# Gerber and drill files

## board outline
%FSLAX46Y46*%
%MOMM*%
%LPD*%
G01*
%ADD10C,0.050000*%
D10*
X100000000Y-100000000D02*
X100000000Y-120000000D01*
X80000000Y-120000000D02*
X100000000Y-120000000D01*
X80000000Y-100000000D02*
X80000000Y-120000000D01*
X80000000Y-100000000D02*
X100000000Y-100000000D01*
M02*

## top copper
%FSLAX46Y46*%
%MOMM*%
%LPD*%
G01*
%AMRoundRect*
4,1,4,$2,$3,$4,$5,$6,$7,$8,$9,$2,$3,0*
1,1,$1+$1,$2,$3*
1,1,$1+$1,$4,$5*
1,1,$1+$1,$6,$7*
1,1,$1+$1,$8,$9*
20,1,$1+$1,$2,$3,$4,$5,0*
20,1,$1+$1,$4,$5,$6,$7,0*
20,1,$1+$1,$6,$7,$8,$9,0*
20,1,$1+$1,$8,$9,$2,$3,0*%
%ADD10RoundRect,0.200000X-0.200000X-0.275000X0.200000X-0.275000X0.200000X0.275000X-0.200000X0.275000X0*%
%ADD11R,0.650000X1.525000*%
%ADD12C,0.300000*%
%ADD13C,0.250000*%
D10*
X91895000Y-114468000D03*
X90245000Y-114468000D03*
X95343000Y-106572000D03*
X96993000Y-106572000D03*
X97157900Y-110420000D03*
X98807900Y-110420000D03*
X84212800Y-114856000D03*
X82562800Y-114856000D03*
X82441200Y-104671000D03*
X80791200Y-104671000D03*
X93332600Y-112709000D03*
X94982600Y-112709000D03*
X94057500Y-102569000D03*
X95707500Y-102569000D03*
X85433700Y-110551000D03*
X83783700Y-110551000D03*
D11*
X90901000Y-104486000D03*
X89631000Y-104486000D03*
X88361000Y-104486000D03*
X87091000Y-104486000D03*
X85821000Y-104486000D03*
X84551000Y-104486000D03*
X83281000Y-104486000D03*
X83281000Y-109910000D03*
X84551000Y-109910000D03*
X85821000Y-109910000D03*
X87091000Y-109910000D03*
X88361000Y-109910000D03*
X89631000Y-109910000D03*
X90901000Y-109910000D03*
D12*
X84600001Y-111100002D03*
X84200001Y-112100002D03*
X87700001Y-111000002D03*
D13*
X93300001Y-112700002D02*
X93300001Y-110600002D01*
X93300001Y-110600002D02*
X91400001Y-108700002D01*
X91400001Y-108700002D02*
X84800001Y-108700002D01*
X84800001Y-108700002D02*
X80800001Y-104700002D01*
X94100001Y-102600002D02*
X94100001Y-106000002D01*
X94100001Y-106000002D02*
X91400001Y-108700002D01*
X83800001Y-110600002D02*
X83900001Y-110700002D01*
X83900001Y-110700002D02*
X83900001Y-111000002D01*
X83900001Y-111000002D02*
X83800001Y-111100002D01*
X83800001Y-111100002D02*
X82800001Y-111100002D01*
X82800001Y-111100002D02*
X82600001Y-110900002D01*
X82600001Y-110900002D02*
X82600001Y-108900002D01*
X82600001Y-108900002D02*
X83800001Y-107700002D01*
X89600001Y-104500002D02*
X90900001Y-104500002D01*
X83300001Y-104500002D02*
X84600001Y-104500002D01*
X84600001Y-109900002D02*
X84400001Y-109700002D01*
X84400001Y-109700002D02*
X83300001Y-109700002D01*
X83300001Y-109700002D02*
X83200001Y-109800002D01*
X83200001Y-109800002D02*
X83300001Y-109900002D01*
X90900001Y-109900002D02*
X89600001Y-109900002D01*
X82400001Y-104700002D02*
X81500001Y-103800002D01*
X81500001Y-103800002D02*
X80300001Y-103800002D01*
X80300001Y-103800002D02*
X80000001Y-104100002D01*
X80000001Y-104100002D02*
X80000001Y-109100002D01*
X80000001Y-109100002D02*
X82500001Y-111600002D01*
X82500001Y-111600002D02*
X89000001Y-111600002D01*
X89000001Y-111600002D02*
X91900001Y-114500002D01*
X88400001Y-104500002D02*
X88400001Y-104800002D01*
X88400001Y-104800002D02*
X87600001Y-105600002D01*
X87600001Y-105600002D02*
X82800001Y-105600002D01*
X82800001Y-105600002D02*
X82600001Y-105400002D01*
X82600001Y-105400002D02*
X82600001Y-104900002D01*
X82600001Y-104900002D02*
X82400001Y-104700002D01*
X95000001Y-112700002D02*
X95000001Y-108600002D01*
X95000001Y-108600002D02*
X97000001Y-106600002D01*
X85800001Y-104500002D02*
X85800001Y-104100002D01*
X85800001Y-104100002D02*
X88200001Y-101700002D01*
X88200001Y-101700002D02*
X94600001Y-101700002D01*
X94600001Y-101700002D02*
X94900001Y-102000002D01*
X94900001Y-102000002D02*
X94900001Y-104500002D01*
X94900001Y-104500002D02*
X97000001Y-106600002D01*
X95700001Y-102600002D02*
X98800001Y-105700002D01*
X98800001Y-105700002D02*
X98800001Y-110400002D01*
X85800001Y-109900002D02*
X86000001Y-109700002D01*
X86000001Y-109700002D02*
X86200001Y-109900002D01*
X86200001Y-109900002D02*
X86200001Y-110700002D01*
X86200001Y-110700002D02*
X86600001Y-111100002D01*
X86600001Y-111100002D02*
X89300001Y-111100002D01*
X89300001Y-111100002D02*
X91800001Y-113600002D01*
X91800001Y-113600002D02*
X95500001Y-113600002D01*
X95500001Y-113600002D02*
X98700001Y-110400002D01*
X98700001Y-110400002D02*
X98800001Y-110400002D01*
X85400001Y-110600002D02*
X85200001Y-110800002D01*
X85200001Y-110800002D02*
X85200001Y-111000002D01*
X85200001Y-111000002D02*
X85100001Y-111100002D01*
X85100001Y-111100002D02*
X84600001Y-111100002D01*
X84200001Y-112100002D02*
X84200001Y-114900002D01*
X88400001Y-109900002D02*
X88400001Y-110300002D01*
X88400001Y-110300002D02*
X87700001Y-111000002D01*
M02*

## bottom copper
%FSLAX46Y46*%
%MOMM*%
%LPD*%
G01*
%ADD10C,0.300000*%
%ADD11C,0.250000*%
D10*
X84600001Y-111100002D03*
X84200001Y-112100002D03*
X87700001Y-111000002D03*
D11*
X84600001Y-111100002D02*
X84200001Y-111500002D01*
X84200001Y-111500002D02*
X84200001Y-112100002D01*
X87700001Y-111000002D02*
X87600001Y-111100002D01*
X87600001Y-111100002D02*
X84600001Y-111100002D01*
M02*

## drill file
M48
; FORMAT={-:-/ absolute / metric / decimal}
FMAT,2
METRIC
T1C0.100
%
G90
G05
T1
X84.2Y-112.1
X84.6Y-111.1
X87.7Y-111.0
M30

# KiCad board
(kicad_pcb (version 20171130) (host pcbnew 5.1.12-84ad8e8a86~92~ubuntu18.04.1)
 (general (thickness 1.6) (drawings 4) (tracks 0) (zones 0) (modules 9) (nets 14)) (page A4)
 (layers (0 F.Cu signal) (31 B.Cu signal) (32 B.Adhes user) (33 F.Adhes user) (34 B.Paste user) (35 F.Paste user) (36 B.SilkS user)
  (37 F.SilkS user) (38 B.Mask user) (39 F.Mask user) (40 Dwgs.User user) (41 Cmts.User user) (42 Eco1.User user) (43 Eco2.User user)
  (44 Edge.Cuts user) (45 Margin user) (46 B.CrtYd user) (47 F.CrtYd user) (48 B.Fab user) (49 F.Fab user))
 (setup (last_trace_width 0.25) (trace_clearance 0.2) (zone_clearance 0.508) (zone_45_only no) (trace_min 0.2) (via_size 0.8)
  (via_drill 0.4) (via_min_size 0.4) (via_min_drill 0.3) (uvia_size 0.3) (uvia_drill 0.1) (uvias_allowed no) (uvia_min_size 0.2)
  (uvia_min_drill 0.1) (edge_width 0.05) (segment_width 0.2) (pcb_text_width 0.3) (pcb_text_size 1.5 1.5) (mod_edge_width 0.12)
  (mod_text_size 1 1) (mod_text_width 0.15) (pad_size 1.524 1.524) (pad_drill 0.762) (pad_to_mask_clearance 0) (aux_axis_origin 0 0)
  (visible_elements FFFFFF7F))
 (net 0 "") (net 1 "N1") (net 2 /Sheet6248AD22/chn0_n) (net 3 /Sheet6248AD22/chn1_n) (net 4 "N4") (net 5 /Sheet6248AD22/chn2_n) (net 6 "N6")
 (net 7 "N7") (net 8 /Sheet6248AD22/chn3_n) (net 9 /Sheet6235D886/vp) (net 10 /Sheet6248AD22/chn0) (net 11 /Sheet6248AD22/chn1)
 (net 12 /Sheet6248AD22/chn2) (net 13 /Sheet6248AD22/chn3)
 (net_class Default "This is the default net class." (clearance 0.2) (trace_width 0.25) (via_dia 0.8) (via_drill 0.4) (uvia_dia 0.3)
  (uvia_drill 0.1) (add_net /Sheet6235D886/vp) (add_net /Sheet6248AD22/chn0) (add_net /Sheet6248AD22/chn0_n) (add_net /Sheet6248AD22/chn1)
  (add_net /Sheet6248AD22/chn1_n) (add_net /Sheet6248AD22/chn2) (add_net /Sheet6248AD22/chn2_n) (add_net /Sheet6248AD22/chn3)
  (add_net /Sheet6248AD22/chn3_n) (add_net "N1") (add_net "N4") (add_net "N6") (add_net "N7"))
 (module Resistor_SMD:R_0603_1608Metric (layer F.Cu) (at 91.070000 114.468000)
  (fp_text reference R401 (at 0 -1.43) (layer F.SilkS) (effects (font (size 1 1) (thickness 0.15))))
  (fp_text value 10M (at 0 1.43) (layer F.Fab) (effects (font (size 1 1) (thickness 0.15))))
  (pad 2 smd roundrect (at 0.825 0) (size 0.8 0.95) (layers F.Cu F.Mask F.Paste) (roundrect_rratio 0.25) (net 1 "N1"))
  (pad 1 smd roundrect (at -0.825 0) (size 0.8 0.95) (layers F.Cu F.Mask F.Paste) (roundrect_rratio 0.25) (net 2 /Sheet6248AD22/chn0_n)))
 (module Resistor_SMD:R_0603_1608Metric (layer F.Cu) (at 96.168000 106.572000)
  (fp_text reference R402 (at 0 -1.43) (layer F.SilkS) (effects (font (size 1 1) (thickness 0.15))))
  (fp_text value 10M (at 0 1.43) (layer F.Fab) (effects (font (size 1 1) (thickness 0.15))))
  (pad 1 smd roundrect (at -0.825 0) (size 0.8 0.95) (layers F.Cu F.Mask F.Paste) (roundrect_rratio 0.25) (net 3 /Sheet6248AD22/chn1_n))
  (pad 2 smd roundrect (at 0.825 0) (size 0.8 0.95) (layers F.Cu F.Mask F.Paste) (roundrect_rratio 0.25) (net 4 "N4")))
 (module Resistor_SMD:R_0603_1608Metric (layer F.Cu) (at 97.982900 110.420000)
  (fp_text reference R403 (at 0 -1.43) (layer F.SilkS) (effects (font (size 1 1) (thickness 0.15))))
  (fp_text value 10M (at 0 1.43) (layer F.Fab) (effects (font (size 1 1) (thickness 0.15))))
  (pad 1 smd roundrect (at -0.825 0) (size 0.8 0.95) (layers F.Cu F.Mask F.Paste) (roundrect_rratio 0.25) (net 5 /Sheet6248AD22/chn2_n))
  (pad 2 smd roundrect (at 0.825 0) (size 0.8 0.95) (layers F.Cu F.Mask F.Paste) (roundrect_rratio 0.25) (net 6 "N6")))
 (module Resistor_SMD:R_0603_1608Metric (layer F.Cu) (at 83.387800 114.856000)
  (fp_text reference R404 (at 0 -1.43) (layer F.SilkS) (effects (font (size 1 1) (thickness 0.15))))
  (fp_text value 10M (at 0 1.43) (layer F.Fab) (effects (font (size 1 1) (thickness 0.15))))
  (pad 2 smd roundrect (at 0.825 0) (size 0.8 0.95) (layers F.Cu F.Mask F.Paste) (roundrect_rratio 0.25) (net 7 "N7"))
  (pad 1 smd roundrect (at -0.825 0) (size 0.8 0.95) (layers F.Cu F.Mask F.Paste) (roundrect_rratio 0.25) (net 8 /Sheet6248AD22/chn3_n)))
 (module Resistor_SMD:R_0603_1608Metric (layer F.Cu) (at 81.616200 104.671000)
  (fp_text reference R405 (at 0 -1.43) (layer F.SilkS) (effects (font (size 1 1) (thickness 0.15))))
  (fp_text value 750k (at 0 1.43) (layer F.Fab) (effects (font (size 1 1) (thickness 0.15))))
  (pad 2 smd roundrect (at 0.825 0) (size 0.8 0.95) (layers F.Cu F.Mask F.Paste) (roundrect_rratio 0.25) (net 1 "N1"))
  (pad 1 smd roundrect (at -0.825 0) (size 0.8 0.95) (layers F.Cu F.Mask F.Paste) (roundrect_rratio 0.25) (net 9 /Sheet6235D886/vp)))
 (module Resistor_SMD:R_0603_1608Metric (layer F.Cu) (at 94.157600 112.709000)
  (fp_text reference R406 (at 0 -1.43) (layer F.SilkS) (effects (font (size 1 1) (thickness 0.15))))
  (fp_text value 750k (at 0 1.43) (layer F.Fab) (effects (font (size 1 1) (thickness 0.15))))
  (pad 1 smd roundrect (at -0.825 0) (size 0.8 0.95) (layers F.Cu F.Mask F.Paste) (roundrect_rratio 0.25) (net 9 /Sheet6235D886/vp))
  (pad 2 smd roundrect (at 0.825 0) (size 0.8 0.95) (layers F.Cu F.Mask F.Paste) (roundrect_rratio 0.25) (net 4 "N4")))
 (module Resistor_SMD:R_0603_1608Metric (layer F.Cu) (at 94.882500 102.569000)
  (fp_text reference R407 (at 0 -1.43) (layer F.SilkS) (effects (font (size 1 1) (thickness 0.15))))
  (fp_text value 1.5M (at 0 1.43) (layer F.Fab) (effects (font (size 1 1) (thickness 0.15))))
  (pad 1 smd roundrect (at -0.825 0) (size 0.8 0.95) (layers F.Cu F.Mask F.Paste) (roundrect_rratio 0.25) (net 9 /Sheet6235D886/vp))
  (pad 2 smd roundrect (at 0.825 0) (size 0.8 0.95) (layers F.Cu F.Mask F.Paste) (roundrect_rratio 0.25) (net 6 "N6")))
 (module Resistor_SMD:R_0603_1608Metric (layer F.Cu) (at 84.608700 110.551000)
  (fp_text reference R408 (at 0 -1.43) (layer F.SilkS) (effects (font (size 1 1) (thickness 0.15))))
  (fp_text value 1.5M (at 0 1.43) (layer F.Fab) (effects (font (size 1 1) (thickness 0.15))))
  (pad 2 smd roundrect (at 0.825 0) (size 0.8 0.95) (layers F.Cu F.Mask F.Paste) (roundrect_rratio 0.25) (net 7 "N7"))
  (pad 1 smd roundrect (at -0.825 0) (size 0.8 0.95) (layers F.Cu F.Mask F.Paste) (roundrect_rratio 0.25) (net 9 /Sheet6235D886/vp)))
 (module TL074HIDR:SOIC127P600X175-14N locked (layer F.Cu) (at 87.091000 107.198000 270.000000)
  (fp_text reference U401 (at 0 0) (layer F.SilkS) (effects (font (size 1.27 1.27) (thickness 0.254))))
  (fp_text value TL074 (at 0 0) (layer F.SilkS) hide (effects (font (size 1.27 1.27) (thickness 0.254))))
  (pad 1 smd rect (at -2.712 -3.81) (size 0.65 1.525) (layers F.Cu F.Mask F.Paste) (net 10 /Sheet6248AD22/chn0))
  (pad 2 smd rect (at -2.712 -2.54) (size 0.65 1.525) (layers F.Cu F.Mask F.Paste) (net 10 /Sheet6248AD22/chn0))
  (pad 3 smd rect (at -2.712 -1.27) (size 0.65 1.525) (layers F.Cu F.Mask F.Paste) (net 1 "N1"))
  (pad 4 smd rect (at -2.712 0) (size 0.65 1.525) (layers F.Cu F.Mask F.Paste))
  (pad 5 smd rect (at -2.712 1.27) (size 0.65 1.525) (layers F.Cu F.Mask F.Paste) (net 4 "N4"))
  (pad 6 smd rect (at -2.712 2.54) (size 0.65 1.525) (layers F.Cu F.Mask F.Paste) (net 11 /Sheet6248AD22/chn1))
  (pad 7 smd rect (at -2.712 3.81) (size 0.65 1.525) (layers F.Cu F.Mask F.Paste) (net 11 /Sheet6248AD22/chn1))
  (pad 8 smd rect (at 2.712 3.81) (size 0.65 1.525) (layers F.Cu F.Mask F.Paste) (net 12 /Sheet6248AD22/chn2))
  (pad 9 smd rect (at 2.712 2.54) (size 0.65 1.525) (layers F.Cu F.Mask F.Paste) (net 12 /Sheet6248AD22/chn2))
  (pad 10 smd rect (at 2.712 1.27) (size 0.65 1.525) (layers F.Cu F.Mask F.Paste) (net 6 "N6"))
  (pad 11 smd rect (at 2.712 0) (size 0.65 1.525) (layers F.Cu F.Mask F.Paste))
  (pad 12 smd rect (at 2.712 -1.27) (size 0.65 1.525) (layers F.Cu F.Mask F.Paste) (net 7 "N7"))
  (pad 13 smd rect (at 2.712 -2.54) (size 0.65 1.525) (layers F.Cu F.Mask F.Paste) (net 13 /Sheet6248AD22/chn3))
  (pad 14 smd rect (at 2.712 -3.81) (size 0.65 1.525) (layers F.Cu F.Mask F.Paste) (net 13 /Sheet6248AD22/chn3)))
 (gr_line (start 100 100) (end 100 120) (layer Edge.Cuts) (width 0.05))
 (gr_line (start 80 120) (end 100 120) (layer Edge.Cuts) (width 0.05))
 (gr_line (start 80 100) (end 80 120) (layer Edge.Cuts) (width 0.05))
 (gr_line (start 80 100) (end 100 100) (layer Edge.Cuts) (width 0.05))
 (segment (start 93.300001 112.700002) (end 93.300001 110.600002) (width 0.250000) (layer F.Cu) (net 9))
 (segment (start 93.300001 110.600002) (end 91.400001 108.700002) (width 0.250000) (layer F.Cu) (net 9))
 (segment (start 91.400001 108.700002) (end 84.800001 108.700002) (width 0.250000) (layer F.Cu) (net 9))
 (segment (start 84.800001 108.700002) (end 80.800001 104.700002) (width 0.250000) (layer F.Cu) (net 9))
 (segment (start 94.100001 102.600002) (end 94.100001 106.000002) (width 0.250000) (layer F.Cu) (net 9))
 (segment (start 94.100001 106.000002) (end 91.400001 108.700002) (width 0.250000) (layer F.Cu) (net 9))
 (segment (start 83.800001 110.600002) (end 83.900001 110.700002) (width 0.250000) (layer F.Cu) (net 9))
 (segment (start 83.900001 110.700002) (end 83.900001 111.000002) (width 0.250000) (layer F.Cu) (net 9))
 (segment (start 83.900001 111.000002) (end 83.800001 111.100002) (width 0.250000) (layer F.Cu) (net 9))
 (segment (start 83.800001 111.100002) (end 82.800001 111.100002) (width 0.250000) (layer F.Cu) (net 9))
 (segment (start 82.800001 111.100002) (end 82.600001 110.900002) (width 0.250000) (layer F.Cu) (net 9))
 (segment (start 82.600001 110.900002) (end 82.600001 108.900002) (width 0.250000) (layer F.Cu) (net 9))
 (segment (start 82.600001 108.900002) (end 83.800001 107.700002) (width 0.250000) (layer F.Cu) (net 9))
 (segment (start 89.600001 104.500002) (end 90.900001 104.500002) (width 0.250000) (layer F.Cu) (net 10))
 (segment (start 83.300001 104.500002) (end 84.600001 104.500002) (width 0.250000) (layer F.Cu) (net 11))
 (segment (start 84.600001 109.900002) (end 84.400001 109.700002) (width 0.250000) (layer F.Cu) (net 12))
 (segment (start 84.400001 109.700002) (end 83.300001 109.700002) (width 0.250000) (layer F.Cu) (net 12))
 (segment (start 83.300001 109.700002) (end 83.200001 109.800002) (width 0.250000) (layer F.Cu) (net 12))
 (segment (start 83.200001 109.800002) (end 83.300001 109.900002) (width 0.250000) (layer F.Cu) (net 12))
 (segment (start 90.900001 109.900002) (end 89.600001 109.900002) (width 0.250000) (layer F.Cu) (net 13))
 (segment (start 82.400001 104.700002) (end 81.500001 103.800002) (width 0.250000) (layer F.Cu) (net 1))
 (segment (start 81.500001 103.800002) (end 80.300001 103.800002) (width 0.250000) (layer F.Cu) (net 1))
 (segment (start 80.300001 103.800002) (end 80.000001 104.100002) (width 0.250000) (layer F.Cu) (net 1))
 (segment (start 80.000001 104.100002) (end 80.000001 109.100002) (width 0.250000) (layer F.Cu) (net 1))
 (segment (start 80.000001 109.100002) (end 82.500001 111.600002) (width 0.250000) (layer F.Cu) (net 1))
 (segment (start 82.500001 111.600002) (end 89.000001 111.600002) (width 0.250000) (layer F.Cu) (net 1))
 (segment (start 89.000001 111.600002) (end 91.900001 114.500002) (width 0.250000) (layer F.Cu) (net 1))
 (segment (start 88.400001 104.500002) (end 88.400001 104.800002) (width 0.250000) (layer F.Cu) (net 1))
 (segment (start 88.400001 104.800002) (end 87.600001 105.600002) (width 0.250000) (layer F.Cu) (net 1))
 (segment (start 87.600001 105.600002) (end 82.800001 105.600002) (width 0.250000) (layer F.Cu) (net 1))
 (segment (start 82.800001 105.600002) (end 82.600001 105.400002) (width 0.250000) (layer F.Cu) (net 1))
 (segment (start 82.600001 105.400002) (end 82.600001 104.900002) (width 0.250000) (layer F.Cu) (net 1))
 (segment (start 82.600001 104.900002) (end 82.400001 104.700002) (width 0.250000) (layer F.Cu) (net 1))
 (segment (start 95.000001 112.700002) (end 95.000001 108.600002) (width 0.250000) (layer F.Cu) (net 4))
 (segment (start 95.000001 108.600002) (end 97.000001 106.600002) (width 0.250000) (layer F.Cu) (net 4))
 (segment (start 85.800001 104.500002) (end 85.800001 104.100002) (width 0.250000) (layer F.Cu) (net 4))
 (segment (start 85.800001 104.100002) (end 88.200001 101.700002) (width 0.250000) (layer F.Cu) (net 4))
 (segment (start 88.200001 101.700002) (end 94.600001 101.700002) (width 0.250000) (layer F.Cu) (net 4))
 (segment (start 94.600001 101.700002) (end 94.900001 102.000002) (width 0.250000) (layer F.Cu) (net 4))
 (segment (start 94.900001 102.000002) (end 94.900001 104.500002) (width 0.250000) (layer F.Cu) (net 4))
 (segment (start 94.900001 104.500002) (end 97.000001 106.600002) (width 0.250000) (layer F.Cu) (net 4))
 (segment (start 95.700001 102.600002) (end 98.800001 105.700002) (width 0.250000) (layer F.Cu) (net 6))
 (segment (start 98.800001 105.700002) (end 98.800001 110.400002) (width 0.250000) (layer F.Cu) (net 6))
 (segment (start 85.800001 109.900002) (end 86.000001 109.700002) (width 0.250000) (layer F.Cu) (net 6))
 (segment (start 86.000001 109.700002) (end 86.200001 109.900002) (width 0.250000) (layer F.Cu) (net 6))
 (segment (start 86.200001 109.900002) (end 86.200001 110.700002) (width 0.250000) (layer F.Cu) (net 6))
 (segment (start 86.200001 110.700002) (end 86.600001 111.100002) (width 0.250000) (layer F.Cu) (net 6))
 (segment (start 86.600001 111.100002) (end 89.300001 111.100002) (width 0.250000) (layer F.Cu) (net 6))
 (segment (start 89.300001 111.100002) (end 91.800001 113.600002) (width 0.250000) (layer F.Cu) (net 6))
 (segment (start 91.800001 113.600002) (end 95.500001 113.600002) (width 0.250000) (layer F.Cu) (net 6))
 (segment (start 95.500001 113.600002) (end 98.700001 110.400002) (width 0.250000) (layer F.Cu) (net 6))
 (segment (start 98.700001 110.400002) (end 98.800001 110.400002) (width 0.250000) (layer F.Cu) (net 6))
 (segment (start 85.400001 110.600002) (end 85.200001 110.800002) (width 0.250000) (layer F.Cu) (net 7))
 (segment (start 85.200001 110.800002) (end 85.200001 111.000002) (width 0.250000) (layer F.Cu) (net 7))
 (segment (start 85.200001 111.000002) (end 85.100001 111.100002) (width 0.250000) (layer F.Cu) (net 7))
 (segment (start 85.100001 111.100002) (end 84.600001 111.100002) (width 0.250000) (layer F.Cu) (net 7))
 (segment (start 84.600001 111.100002) (end 84.200001 111.500002) (width 0.250000) (layer B.Cu) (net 7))
 (segment (start 84.200001 111.500002) (end 84.200001 112.100002) (width 0.250000) (layer B.Cu) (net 7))
 (segment (start 84.200001 112.100002) (end 84.200001 114.900002) (width 0.250000) (layer F.Cu) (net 7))
 (segment (start 88.400001 109.900002) (end 88.400001 110.300002) (width 0.250000) (layer F.Cu) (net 7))
 (segment (start 88.400001 110.300002) (end 87.700001 111.000002) (width 0.250000) (layer F.Cu) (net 7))
 (segment (start 87.700001 111.000002) (end 87.600001 111.100002) (width 0.250000) (layer B.Cu) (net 7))
 (segment (start 87.600001 111.100002) (end 84.600001 111.100002) (width 0.250000) (layer B.Cu) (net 7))
 (via micro (at 84.600001 111.100002) (size 0.300000) (drill 0.100000) (layers F.Cu B.Cu) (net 7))
 (via micro (at 84.200001 112.100002) (size 0.300000) (drill 0.100000) (layers F.Cu B.Cu) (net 7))
 (via micro (at 87.700001 111.000002) (size 0.300000) (drill 0.100000) (layers F.Cu B.Cu) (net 7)))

